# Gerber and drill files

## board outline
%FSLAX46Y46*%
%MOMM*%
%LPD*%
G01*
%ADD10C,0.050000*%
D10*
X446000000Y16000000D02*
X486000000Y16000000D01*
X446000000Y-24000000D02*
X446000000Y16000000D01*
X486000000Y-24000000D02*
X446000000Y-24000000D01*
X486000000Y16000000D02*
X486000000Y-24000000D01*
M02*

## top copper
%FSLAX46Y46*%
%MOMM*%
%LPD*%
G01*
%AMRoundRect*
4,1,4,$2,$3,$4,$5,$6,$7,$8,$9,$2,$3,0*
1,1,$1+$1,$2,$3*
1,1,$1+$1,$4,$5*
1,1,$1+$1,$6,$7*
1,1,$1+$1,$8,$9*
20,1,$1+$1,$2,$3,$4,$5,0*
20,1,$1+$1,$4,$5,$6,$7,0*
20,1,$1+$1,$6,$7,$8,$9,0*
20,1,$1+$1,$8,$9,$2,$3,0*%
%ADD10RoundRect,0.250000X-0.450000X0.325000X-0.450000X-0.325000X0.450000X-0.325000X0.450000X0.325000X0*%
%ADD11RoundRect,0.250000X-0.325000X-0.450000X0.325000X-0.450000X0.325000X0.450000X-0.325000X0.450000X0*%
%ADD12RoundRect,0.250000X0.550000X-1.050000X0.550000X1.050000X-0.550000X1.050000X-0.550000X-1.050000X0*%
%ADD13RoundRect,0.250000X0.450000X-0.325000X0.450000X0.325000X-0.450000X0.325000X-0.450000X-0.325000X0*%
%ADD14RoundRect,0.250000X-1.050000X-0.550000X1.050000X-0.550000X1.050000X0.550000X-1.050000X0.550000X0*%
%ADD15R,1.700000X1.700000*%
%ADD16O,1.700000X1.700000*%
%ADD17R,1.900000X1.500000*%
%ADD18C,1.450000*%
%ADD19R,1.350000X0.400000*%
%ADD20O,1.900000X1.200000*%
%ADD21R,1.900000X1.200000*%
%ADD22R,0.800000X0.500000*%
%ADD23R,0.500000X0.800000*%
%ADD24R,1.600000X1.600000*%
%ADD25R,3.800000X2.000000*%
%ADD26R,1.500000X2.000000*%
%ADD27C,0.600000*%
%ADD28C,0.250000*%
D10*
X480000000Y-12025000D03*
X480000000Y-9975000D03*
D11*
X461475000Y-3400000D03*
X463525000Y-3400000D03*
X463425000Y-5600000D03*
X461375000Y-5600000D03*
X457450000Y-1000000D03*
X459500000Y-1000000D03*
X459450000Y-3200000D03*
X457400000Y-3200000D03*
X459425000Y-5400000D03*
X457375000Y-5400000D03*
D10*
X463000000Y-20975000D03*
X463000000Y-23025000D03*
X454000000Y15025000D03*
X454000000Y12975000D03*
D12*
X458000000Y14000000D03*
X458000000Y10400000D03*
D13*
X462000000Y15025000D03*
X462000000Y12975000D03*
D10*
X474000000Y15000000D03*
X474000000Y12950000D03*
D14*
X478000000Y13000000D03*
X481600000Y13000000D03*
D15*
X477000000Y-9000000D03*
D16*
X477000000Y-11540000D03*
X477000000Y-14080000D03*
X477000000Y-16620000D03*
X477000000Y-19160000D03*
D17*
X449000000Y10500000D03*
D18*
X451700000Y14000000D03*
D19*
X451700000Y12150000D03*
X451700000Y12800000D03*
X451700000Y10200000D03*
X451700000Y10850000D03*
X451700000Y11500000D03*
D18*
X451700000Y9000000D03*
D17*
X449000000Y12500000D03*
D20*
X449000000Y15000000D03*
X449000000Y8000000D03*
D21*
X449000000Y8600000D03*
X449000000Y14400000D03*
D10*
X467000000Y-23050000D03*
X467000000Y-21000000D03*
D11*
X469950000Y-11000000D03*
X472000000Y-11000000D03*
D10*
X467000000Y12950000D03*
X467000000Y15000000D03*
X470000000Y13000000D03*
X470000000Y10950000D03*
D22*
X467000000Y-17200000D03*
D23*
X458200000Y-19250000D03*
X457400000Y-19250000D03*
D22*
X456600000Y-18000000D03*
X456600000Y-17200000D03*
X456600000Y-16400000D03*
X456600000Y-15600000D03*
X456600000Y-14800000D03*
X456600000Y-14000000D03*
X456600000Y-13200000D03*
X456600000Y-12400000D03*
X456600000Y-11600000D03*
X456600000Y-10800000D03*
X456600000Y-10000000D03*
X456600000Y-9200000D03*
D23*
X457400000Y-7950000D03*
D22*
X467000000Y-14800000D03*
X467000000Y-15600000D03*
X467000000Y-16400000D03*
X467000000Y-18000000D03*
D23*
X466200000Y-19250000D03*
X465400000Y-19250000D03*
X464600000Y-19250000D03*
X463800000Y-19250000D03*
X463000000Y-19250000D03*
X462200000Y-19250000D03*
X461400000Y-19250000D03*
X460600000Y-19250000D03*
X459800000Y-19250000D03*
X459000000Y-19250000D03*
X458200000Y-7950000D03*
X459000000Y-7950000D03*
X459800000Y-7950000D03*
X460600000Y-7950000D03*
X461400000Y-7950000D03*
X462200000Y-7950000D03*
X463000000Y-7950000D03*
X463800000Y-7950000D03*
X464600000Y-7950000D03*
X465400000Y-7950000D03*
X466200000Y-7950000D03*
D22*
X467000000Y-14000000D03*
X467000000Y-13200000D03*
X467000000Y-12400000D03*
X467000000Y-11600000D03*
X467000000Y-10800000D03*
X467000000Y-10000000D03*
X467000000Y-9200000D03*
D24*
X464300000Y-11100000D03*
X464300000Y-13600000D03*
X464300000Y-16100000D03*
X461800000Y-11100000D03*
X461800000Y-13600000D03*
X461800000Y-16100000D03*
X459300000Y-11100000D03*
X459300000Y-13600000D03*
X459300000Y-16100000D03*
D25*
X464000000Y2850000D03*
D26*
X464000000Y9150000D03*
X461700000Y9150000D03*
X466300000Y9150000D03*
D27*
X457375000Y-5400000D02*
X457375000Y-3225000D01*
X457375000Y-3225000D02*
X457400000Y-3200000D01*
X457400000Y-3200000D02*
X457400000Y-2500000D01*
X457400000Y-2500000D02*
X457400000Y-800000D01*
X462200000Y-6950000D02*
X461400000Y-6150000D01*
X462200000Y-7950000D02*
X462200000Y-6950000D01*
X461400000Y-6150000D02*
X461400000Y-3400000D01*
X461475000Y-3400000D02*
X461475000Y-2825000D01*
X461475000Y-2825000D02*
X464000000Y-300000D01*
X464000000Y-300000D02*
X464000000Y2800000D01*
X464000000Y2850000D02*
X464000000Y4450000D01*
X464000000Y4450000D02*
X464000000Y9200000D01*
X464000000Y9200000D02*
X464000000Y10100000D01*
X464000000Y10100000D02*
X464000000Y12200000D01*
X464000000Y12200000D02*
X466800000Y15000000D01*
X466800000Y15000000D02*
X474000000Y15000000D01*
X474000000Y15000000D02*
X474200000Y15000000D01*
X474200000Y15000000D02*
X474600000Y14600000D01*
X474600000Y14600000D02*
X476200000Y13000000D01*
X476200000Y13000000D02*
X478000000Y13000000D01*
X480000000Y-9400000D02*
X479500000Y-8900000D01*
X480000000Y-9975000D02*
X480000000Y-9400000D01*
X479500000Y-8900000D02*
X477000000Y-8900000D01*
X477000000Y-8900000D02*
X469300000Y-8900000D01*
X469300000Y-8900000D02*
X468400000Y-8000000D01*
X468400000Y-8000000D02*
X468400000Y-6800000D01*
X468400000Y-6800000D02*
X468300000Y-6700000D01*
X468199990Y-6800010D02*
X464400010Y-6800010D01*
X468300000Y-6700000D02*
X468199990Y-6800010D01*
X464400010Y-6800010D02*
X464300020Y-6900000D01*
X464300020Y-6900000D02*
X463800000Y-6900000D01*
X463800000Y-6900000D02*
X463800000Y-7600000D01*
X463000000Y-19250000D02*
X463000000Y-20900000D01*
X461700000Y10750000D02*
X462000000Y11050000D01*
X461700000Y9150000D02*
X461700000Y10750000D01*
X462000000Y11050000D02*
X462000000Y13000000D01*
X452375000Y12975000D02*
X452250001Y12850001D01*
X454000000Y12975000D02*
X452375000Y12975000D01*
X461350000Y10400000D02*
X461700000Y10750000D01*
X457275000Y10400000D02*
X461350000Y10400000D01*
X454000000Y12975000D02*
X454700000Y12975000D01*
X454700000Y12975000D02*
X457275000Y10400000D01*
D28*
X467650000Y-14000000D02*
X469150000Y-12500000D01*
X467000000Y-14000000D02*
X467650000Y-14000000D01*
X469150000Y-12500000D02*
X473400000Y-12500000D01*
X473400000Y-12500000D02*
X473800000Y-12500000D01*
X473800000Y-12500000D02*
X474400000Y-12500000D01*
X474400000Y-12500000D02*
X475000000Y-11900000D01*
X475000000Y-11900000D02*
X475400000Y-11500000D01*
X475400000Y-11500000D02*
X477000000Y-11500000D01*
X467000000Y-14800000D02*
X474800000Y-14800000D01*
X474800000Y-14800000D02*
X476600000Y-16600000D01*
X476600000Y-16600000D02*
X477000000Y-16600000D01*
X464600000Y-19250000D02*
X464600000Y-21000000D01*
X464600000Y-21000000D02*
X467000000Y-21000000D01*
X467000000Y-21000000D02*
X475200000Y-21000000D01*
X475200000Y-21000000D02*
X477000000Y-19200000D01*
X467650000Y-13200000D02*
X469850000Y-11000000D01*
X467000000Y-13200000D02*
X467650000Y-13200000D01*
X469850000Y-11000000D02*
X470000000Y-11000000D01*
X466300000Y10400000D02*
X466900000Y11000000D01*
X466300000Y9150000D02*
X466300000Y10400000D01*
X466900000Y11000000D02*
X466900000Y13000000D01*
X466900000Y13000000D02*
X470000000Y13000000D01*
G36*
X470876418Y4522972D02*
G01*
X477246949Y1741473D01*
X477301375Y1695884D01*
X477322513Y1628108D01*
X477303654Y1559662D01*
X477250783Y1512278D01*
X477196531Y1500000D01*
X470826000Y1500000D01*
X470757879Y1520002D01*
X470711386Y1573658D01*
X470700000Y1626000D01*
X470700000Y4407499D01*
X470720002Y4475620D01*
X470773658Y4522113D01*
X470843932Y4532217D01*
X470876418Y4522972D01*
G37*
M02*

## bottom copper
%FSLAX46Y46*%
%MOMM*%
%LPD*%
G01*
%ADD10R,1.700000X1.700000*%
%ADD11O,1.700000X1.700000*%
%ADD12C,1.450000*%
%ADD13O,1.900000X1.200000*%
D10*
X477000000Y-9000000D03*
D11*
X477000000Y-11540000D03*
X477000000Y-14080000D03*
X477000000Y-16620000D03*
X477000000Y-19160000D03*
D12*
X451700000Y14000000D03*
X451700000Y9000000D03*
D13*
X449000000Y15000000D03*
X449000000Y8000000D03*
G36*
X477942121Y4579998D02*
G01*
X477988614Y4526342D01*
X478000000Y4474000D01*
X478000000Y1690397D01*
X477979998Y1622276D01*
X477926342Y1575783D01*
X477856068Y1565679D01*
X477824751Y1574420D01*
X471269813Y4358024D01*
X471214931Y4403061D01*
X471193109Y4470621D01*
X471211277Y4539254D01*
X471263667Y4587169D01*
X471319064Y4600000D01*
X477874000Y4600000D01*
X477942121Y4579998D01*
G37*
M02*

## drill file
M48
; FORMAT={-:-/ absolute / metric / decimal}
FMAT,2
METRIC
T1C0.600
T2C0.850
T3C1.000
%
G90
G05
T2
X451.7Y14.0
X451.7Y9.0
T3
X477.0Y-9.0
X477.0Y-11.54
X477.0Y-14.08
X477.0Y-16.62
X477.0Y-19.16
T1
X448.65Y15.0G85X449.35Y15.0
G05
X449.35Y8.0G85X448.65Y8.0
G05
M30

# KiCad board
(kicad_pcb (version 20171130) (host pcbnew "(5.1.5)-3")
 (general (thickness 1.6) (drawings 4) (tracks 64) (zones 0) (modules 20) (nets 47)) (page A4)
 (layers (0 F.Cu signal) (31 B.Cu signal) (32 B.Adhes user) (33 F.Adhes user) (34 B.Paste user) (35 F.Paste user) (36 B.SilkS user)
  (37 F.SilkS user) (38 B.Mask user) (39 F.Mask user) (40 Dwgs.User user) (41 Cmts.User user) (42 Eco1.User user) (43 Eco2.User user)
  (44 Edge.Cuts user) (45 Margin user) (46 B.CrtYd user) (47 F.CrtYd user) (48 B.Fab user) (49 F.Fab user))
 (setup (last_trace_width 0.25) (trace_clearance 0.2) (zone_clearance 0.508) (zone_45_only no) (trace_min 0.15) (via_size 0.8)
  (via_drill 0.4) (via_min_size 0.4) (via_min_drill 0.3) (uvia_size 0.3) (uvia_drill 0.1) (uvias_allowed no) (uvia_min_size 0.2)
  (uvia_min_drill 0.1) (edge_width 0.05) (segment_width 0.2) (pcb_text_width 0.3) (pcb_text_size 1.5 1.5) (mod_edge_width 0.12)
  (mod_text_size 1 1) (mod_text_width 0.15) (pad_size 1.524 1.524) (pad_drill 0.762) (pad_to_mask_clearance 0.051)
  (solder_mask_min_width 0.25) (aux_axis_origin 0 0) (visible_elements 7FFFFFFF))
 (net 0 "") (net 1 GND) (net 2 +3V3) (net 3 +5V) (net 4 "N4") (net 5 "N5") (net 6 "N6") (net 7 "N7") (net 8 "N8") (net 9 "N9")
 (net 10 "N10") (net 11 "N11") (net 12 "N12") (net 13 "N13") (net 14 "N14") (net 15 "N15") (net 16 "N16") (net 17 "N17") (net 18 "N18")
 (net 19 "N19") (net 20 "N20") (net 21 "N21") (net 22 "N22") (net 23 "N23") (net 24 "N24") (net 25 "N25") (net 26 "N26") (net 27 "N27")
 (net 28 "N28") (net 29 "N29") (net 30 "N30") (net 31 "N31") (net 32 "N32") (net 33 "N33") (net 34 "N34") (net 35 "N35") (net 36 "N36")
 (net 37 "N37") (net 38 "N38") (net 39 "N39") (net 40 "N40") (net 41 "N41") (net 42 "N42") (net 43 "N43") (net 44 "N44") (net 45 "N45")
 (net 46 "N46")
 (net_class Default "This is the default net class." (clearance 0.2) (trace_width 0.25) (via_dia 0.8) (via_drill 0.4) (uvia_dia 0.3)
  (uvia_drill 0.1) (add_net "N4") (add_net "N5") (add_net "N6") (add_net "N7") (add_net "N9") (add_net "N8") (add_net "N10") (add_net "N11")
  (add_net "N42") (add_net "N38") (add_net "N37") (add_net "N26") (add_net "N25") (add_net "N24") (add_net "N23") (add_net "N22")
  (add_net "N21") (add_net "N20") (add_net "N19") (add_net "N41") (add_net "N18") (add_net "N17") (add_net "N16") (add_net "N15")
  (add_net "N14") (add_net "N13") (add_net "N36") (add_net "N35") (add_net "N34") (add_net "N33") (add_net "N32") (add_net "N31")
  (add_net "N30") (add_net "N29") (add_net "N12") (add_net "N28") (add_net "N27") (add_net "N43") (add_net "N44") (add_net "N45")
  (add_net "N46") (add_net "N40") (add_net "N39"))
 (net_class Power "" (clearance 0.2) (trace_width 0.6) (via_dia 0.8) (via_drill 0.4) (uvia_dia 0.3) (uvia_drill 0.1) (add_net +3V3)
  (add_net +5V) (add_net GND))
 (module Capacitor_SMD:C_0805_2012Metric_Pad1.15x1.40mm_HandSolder (layer F.Cu) (at 480 11 270)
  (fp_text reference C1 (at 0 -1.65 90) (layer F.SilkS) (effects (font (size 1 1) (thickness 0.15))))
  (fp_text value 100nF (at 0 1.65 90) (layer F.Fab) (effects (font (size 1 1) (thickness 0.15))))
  (pad 2 smd roundrect (at 1.025 0 270) (size 1.15 1.4) (layers F.Cu F.Paste F.Mask) (roundrect_rratio 0.217391) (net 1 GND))
  (pad 1 smd roundrect (at -1.025 0 270) (size 1.15 1.4) (layers F.Cu F.Paste F.Mask) (roundrect_rratio 0.217391) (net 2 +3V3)))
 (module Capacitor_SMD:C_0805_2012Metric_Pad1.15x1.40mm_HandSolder (layer F.Cu) (at 462.5 3.4)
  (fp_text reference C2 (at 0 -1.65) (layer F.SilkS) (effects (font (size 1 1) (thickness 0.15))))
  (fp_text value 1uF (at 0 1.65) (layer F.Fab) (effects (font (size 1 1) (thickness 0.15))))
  (pad 1 smd roundrect (at -1.025 0) (size 1.15 1.4) (layers F.Cu F.Paste F.Mask) (roundrect_rratio 0.217391) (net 2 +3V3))
  (pad 2 smd roundrect (at 1.025 0) (size 1.15 1.4) (layers F.Cu F.Paste F.Mask) (roundrect_rratio 0.217391) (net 1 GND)))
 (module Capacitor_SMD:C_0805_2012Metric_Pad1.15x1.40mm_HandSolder (layer F.Cu) (at 462.4 5.6)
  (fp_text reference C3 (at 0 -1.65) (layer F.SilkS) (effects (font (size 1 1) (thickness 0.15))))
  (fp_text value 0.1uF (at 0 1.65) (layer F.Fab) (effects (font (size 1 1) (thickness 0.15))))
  (pad 2 smd roundrect (at 1.025 0) (size 1.15 1.4) (layers F.Cu F.Paste F.Mask) (roundrect_rratio 0.217391) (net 1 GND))
  (pad 1 smd roundrect (at -1.025 0) (size 1.15 1.4) (layers F.Cu F.Paste F.Mask) (roundrect_rratio 0.217391) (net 2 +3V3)))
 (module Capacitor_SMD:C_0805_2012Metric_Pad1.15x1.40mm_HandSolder (layer F.Cu) (at 458.475 1)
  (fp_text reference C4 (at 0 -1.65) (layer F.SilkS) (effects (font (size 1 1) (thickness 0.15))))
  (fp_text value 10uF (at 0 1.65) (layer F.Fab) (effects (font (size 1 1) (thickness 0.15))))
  (pad 1 smd roundrect (at -1.025 0) (size 1.15 1.4) (layers F.Cu F.Paste F.Mask) (roundrect_rratio 0.217391) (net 2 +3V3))
  (pad 2 smd roundrect (at 1.025 0) (size 1.15 1.4) (layers F.Cu F.Paste F.Mask) (roundrect_rratio 0.217391) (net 1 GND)))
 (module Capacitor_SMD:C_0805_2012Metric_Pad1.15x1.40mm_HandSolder (layer F.Cu) (at 458.425 3.2)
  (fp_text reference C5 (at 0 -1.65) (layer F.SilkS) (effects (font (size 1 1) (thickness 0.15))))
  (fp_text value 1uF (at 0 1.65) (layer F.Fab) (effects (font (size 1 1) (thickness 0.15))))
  (pad 2 smd roundrect (at 1.025 0) (size 1.15 1.4) (layers F.Cu F.Paste F.Mask) (roundrect_rratio 0.217391) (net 1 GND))
  (pad 1 smd roundrect (at -1.025 0) (size 1.15 1.4) (layers F.Cu F.Paste F.Mask) (roundrect_rratio 0.217391) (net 2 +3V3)))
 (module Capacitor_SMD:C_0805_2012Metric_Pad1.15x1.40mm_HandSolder (layer F.Cu) (at 458.4 5.4)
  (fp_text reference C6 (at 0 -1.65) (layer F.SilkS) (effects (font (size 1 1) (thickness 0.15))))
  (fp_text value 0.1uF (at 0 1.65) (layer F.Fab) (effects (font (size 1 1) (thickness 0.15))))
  (pad 2 smd roundrect (at 1.025 0) (size 1.15 1.4) (layers F.Cu F.Paste F.Mask) (roundrect_rratio 0.217391) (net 1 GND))
  (pad 1 smd roundrect (at -1.025 0) (size 1.15 1.4) (layers F.Cu F.Paste F.Mask) (roundrect_rratio 0.217391) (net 2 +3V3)))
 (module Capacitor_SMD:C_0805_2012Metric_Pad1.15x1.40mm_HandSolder (layer F.Cu) (at 463 22 270)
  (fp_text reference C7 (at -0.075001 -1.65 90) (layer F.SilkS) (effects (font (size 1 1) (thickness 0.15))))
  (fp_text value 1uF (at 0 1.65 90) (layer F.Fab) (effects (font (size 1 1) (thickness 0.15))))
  (pad 1 smd roundrect (at -1.025 0 270) (size 1.15 1.4) (layers F.Cu F.Paste F.Mask) (roundrect_rratio 0.217391) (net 2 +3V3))
  (pad 2 smd roundrect (at 1.025 0 270) (size 1.15 1.4) (layers F.Cu F.Paste F.Mask) (roundrect_rratio 0.217391) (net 1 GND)))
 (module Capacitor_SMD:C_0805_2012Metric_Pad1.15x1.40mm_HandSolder (layer F.Cu) (at 454 -14 270)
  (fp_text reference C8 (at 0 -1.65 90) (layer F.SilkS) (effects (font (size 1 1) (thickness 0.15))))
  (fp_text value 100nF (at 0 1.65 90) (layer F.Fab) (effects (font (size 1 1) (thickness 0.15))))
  (pad 1 smd roundrect (at -1.025 0 270) (size 1.15 1.4) (layers F.Cu F.Paste F.Mask) (roundrect_rratio 0.217391) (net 1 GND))
  (pad 2 smd roundrect (at 1.025 0 270) (size 1.15 1.4) (layers F.Cu F.Paste F.Mask) (roundrect_rratio 0.217391) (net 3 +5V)))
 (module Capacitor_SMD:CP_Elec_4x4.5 (layer F.Cu) (at 458 -12.2 90)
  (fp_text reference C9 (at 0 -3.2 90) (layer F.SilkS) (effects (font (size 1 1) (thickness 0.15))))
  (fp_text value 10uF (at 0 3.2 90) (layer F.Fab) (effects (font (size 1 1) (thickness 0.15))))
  (pad 2 smd roundrect (at 1.8 0 90) (size 2.6 1.6) (layers F.Cu F.Paste F.Mask) (roundrect_rratio 0.15625) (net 1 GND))
  (pad 1 smd roundrect (at -1.8 0 90) (size 2.6 1.6) (layers F.Cu F.Paste F.Mask) (roundrect_rratio 0.15625) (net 3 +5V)))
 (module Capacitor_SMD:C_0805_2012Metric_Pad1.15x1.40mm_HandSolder (layer F.Cu) (at 462 -14 90)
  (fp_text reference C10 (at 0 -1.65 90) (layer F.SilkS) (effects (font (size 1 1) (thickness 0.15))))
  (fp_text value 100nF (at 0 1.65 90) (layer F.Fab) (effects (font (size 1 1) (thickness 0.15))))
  (pad 2 smd roundrect (at 1.025 0 90) (size 1.15 1.4) (layers F.Cu F.Paste F.Mask) (roundrect_rratio 0.217391) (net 1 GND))
  (pad 1 smd roundrect (at -1.025 0 90) (size 1.15 1.4) (layers F.Cu F.Paste F.Mask) (roundrect_rratio 0.217391) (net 3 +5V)))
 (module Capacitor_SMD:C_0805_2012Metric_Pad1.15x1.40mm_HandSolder (layer F.Cu) (at 474 -13.975 270)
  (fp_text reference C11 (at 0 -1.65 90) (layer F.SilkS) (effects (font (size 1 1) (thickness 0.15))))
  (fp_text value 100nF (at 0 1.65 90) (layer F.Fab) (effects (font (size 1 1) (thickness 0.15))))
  (pad 1 smd roundrect (at -1.025 0 270) (size 1.15 1.4) (layers F.Cu F.Paste F.Mask) (roundrect_rratio 0.217391) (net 2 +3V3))
  (pad 2 smd roundrect (at 1.025 0 270) (size 1.15 1.4) (layers F.Cu F.Paste F.Mask) (roundrect_rratio 0.217391) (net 1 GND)))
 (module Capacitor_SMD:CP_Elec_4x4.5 (layer F.Cu) (at 479.8 -13)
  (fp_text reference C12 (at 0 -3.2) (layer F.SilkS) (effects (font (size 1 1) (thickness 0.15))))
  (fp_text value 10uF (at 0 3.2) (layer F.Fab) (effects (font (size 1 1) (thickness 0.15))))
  (pad 1 smd roundrect (at -1.8 0) (size 2.6 1.6) (layers F.Cu F.Paste F.Mask) (roundrect_rratio 0.15625) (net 2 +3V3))
  (pad 2 smd roundrect (at 1.8 0) (size 2.6 1.6) (layers F.Cu F.Paste F.Mask) (roundrect_rratio 0.15625) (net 1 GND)))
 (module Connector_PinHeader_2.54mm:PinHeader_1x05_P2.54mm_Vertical (layer F.Cu) (at 477 9)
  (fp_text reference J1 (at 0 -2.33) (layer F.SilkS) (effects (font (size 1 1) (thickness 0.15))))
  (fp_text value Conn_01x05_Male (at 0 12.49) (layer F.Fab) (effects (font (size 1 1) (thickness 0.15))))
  (pad 1 thru_hole rect (at 0 0) (size 1.7 1.7) (drill 1) (layers *.Cu *.Mask) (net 2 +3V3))
  (pad 2 thru_hole oval (at 0 2.54) (size 1.7 1.7) (drill 1) (layers *.Cu *.Mask) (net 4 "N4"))
  (pad 3 thru_hole oval (at 0 5.08) (size 1.7 1.7) (drill 1) (layers *.Cu *.Mask) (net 1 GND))
  (pad 4 thru_hole oval (at 0 7.62) (size 1.7 1.7) (drill 1) (layers *.Cu *.Mask) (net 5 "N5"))
  (pad 5 thru_hole oval (at 0 10.16) (size 1.7 1.7) (drill 1) (layers *.Cu *.Mask) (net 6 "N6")))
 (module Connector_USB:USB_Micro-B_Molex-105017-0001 (layer F.Cu) (at 450.2375 -11.5 270)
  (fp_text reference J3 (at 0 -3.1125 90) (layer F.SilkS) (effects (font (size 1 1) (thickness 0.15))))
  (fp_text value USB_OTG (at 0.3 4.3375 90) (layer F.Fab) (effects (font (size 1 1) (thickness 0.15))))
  (pad 6 smd rect (at 1 1.2375 270) (size 1.5 1.9) (layers F.Cu F.Paste F.Mask) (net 1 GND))
  (pad 6 thru_hole circle (at -2.5 -1.4625 270) (size 1.45 1.45) (drill 0.85) (layers *.Cu *.Mask) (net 1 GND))
  (pad 2 smd rect (at -0.65 -1.4625 270) (size 0.4 1.35) (layers F.Cu F.Paste F.Mask) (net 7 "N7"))
  (pad 1 smd rect (at -1.3 -1.4625 270) (size 0.4 1.35) (layers F.Cu F.Paste F.Mask) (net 3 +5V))
  (pad 5 smd rect (at 1.3 -1.4625 270) (size 0.4 1.35) (layers F.Cu F.Paste F.Mask) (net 1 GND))
  (pad 4 smd rect (at 0.65 -1.4625 270) (size 0.4 1.35) (layers F.Cu F.Paste F.Mask) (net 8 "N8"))
  (pad 3 smd rect (at 0 -1.4625 270) (size 0.4 1.35) (layers F.Cu F.Paste F.Mask) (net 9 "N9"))
  (pad 6 thru_hole circle (at 2.5 -1.4625 270) (size 1.45 1.45) (drill 0.85) (layers *.Cu *.Mask) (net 1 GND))
  (pad 6 smd rect (at -1 1.2375 270) (size 1.5 1.9) (layers F.Cu F.Paste F.Mask) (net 1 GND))
  (pad 6 thru_hole oval (at -3.5 1.2375 90) (size 1.2 1.9) (drill oval 0.6 1.3) (layers *.Cu *.Mask) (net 1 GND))
  (pad 6 thru_hole oval (at 3.5 1.2375 270) (size 1.2 1.9) (drill oval 0.6 1.3) (layers *.Cu *.Mask) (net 1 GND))
  (pad 6 smd rect (at 2.9 1.2375 270) (size 1.2 1.9) (layers F.Cu F.Mask) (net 1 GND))
  (pad 6 smd rect (at -2.9 1.2375 270) (size 1.2 1.9) (layers F.Cu F.Mask) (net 1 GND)))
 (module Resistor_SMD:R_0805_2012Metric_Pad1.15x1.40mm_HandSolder (layer F.Cu) (at 467 22.025 270)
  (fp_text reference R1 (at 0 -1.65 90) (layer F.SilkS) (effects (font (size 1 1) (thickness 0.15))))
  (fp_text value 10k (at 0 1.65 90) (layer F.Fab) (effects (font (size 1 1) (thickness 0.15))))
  (pad 2 smd roundrect (at 1.025 0 270) (size 1.15 1.4) (layers F.Cu F.Paste F.Mask) (roundrect_rratio 0.217391) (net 1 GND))
  (pad 1 smd roundrect (at -1.025 0 270) (size 1.15 1.4) (layers F.Cu F.Paste F.Mask) (roundrect_rratio 0.217391) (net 6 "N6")))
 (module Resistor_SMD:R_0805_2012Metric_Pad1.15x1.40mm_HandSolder (layer F.Cu) (at 470.975 11)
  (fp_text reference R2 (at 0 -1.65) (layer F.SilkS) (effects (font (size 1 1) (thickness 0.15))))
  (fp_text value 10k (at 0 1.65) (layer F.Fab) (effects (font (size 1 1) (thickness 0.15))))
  (pad 1 smd roundrect (at -1.025 0) (size 1.15 1.4) (layers F.Cu F.Paste F.Mask) (roundrect_rratio 0.217391) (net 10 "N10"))
  (pad 2 smd roundrect (at 1.025 0) (size 1.15 1.4) (layers F.Cu F.Paste F.Mask) (roundrect_rratio 0.217391) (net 1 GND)))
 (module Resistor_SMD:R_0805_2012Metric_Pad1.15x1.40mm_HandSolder (layer F.Cu) (at 467 -13.975 270)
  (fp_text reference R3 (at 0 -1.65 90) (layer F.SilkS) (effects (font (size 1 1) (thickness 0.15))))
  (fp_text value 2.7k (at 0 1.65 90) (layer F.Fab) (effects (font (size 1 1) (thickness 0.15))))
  (pad 2 smd roundrect (at 1.025 0 270) (size 1.15 1.4) (layers F.Cu F.Paste F.Mask) (roundrect_rratio 0.217391) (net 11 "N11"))
  (pad 1 smd roundrect (at -1.025 0 270) (size 1.15 1.4) (layers F.Cu F.Paste F.Mask) (roundrect_rratio 0.217391) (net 2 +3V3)))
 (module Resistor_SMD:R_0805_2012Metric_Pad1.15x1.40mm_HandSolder (layer F.Cu) (at 470 -11.975 270)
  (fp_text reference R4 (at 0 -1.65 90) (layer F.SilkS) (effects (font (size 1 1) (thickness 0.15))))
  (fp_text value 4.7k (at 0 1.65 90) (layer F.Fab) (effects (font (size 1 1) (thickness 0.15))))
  (pad 1 smd roundrect (at -1.025 0 270) (size 1.15 1.4) (layers F.Cu F.Paste F.Mask) (roundrect_rratio 0.217391) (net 11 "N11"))
  (pad 2 smd roundrect (at 1.025 0 270) (size 1.15 1.4) (layers F.Cu F.Paste F.Mask) (roundrect_rratio 0.217391) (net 1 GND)))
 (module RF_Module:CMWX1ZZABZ (layer F.Cu) (at 461.8 13.6 270)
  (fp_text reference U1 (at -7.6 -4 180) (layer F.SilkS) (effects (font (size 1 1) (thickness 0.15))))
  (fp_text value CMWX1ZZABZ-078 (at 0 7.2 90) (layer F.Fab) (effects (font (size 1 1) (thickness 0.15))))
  (pad 38 smd rect (at 3.6 -5.2) (size 0.8 0.5) (layers F.Cu F.Paste F.Mask) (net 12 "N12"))
  (pad 26 smd rect (at 5.65 3.6 270) (size 0.8 0.5) (layers F.Cu F.Paste F.Mask) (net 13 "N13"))
  (pad 25 smd rect (at 5.65 4.4 270) (size 0.8 0.5) (layers F.Cu F.Paste F.Mask) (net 1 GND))
  (pad 24 smd rect (at 4.4 5.2 180) (size 0.8 0.5) (layers F.Cu F.Paste F.Mask) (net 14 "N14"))
  (pad 23 smd rect (at 3.6 5.2 180) (size 0.8 0.5) (layers F.Cu F.Paste F.Mask) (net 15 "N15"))
  (pad 22 smd rect (at 2.8 5.2 180) (size 0.8 0.5) (layers F.Cu F.Paste F.Mask) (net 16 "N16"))
  (pad 21 smd rect (at 2 5.2 180) (size 0.8 0.5) (layers F.Cu F.Paste F.Mask) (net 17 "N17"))
  (pad 20 smd rect (at 1.2 5.2 180) (size 0.8 0.5) (layers F.Cu F.Paste F.Mask) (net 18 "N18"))
  (pad 19 smd rect (at 0.4 5.2) (size 0.8 0.5) (layers F.Cu F.Paste F.Mask) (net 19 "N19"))
  (pad 18 smd rect (at -0.4 5.2) (size 0.8 0.5) (layers F.Cu F.Paste F.Mask) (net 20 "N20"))
  (pad 17 smd rect (at -1.2 5.2) (size 0.8 0.5) (layers F.Cu F.Paste F.Mask) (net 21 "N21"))
  (pad 16 smd rect (at -2 5.2) (size 0.8 0.5) (layers F.Cu F.Paste F.Mask) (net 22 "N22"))
  (pad 15 smd rect (at -2.8 5.2) (size 0.8 0.5) (layers F.Cu F.Paste F.Mask) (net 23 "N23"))
  (pad 14 smd rect (at -3.6 5.2) (size 0.8 0.5) (layers F.Cu F.Paste F.Mask) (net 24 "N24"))
  (pad 13 smd rect (at -4.4 5.2) (size 0.8 0.5) (layers F.Cu F.Paste F.Mask) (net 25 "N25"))
  (pad 12 smd rect (at -5.65 4.4 270) (size 0.8 0.5) (layers F.Cu F.Paste F.Mask) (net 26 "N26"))
  (pad 41 smd rect (at 1.2 -5.2) (size 0.8 0.5) (layers F.Cu F.Paste F.Mask) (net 5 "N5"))
  (pad 40 smd rect (at 2 -5.2) (size 0.8 0.5) (layers F.Cu F.Paste F.Mask) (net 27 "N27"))
  (pad 39 smd rect (at 2.8 -5.2) (size 0.8 0.5) (layers F.Cu F.Paste F.Mask) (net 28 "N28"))
  (pad 37 smd rect (at 4.4 -5.2) (size 0.8 0.5) (layers F.Cu F.Paste F.Mask) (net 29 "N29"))
  (pad 36 smd rect (at 5.65 -4.4 270) (size 0.8 0.5) (layers F.Cu F.Paste F.Mask) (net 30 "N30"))
  (pad 35 smd rect (at 5.65 -3.6 270) (size 0.8 0.5) (layers F.Cu F.Paste F.Mask) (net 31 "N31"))
  (pad 34 smd rect (at 5.65 -2.8 270) (size 0.8 0.5) (layers F.Cu F.Paste F.Mask) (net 6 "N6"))
  (pad 33 smd rect (at 5.65 -2 270) (size 0.8 0.5) (layers F.Cu F.Paste F.Mask) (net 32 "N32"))
  (pad 32 smd rect (at 5.65 -1.2 270) (size 0.8 0.5) (layers F.Cu F.Paste F.Mask) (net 2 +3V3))
  (pad 31 smd rect (at 5.65 -0.4 270) (size 0.8 0.5) (layers F.Cu F.Paste F.Mask) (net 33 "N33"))
  (pad 30 smd rect (at 5.65 0.4 270) (size 0.8 0.5) (layers F.Cu F.Paste F.Mask) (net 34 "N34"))
  (pad 29 smd rect (at 5.65 1.2 270) (size 0.8 0.5) (layers F.Cu F.Paste F.Mask) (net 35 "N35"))
  (pad 28 smd rect (at 5.65 2 270) (size 0.8 0.5) (layers F.Cu F.Paste F.Mask) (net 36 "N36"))
  (pad 27 smd rect (at 5.65 2.8 270) (size 0.8 0.5) (layers F.Cu F.Paste F.Mask) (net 1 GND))
  (pad 11 smd rect (at -5.65 3.6 270) (size 0.8 0.5) (layers F.Cu F.Paste F.Mask) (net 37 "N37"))
  (pad 10 smd rect (at -5.65 2.8 270) (size 0.8 0.5) (layers F.Cu F.Paste F.Mask) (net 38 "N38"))
  (pad 9 smd rect (at -5.65 2 270) (size 0.8 0.5) (layers F.Cu F.Paste F.Mask) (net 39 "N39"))
  (pad 8 smd rect (at -5.65 1.2 270) (size 0.8 0.5) (layers F.Cu F.Paste F.Mask) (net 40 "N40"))
  (pad 7 smd rect (at -5.65 0.4 270) (size 0.8 0.5) (layers F.Cu F.Paste F.Mask) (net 1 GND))
  (pad 6 smd rect (at -5.65 -0.4 270) (size 0.8 0.5) (layers F.Cu F.Paste F.Mask) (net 2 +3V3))
  (pad 5 smd rect (at -5.65 -1.2 270) (size 0.8 0.5) (layers F.Cu F.Paste F.Mask) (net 2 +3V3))
  (pad 4 smd rect (at -5.65 -2 270) (size 0.8 0.5) (layers F.Cu F.Paste F.Mask) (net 2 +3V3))
  (pad 3 smd rect (at -5.65 -2.8 270) (size 0.8 0.5) (layers F.Cu F.Paste F.Mask) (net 1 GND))
  (pad 2 smd rect (at -5.65 -3.6 270) (size 0.8 0.5) (layers F.Cu F.Paste F.Mask) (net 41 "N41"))
  (pad 1 smd rect (at -5.65 -4.4 270) (size 0.8 0.5) (layers F.Cu F.Paste F.Mask) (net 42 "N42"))
  (pad 42 smd rect (at 0.4 -5.2) (size 0.8 0.5) (layers F.Cu F.Paste F.Mask) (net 4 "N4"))
  (pad 43 smd rect (at -0.4 -5.2) (size 0.8 0.5) (layers F.Cu F.Paste F.Mask) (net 10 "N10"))
  (pad 44 smd rect (at -1.2 -5.2) (size 0.8 0.5) (layers F.Cu F.Paste F.Mask) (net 1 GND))
  (pad 45 smd rect (at -2 -5.2) (size 0.8 0.5) (layers F.Cu F.Paste F.Mask) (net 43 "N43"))
  (pad 46 smd rect (at -2.8 -5.2) (size 0.8 0.5) (layers F.Cu F.Paste F.Mask) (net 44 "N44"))
  (pad 47 smd rect (at -3.6 -5.2) (size 0.8 0.5) (layers F.Cu F.Paste F.Mask) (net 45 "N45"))
  (pad 48 smd rect (at -4.4 -5.2) (size 0.8 0.5) (layers F.Cu F.Paste F.Mask) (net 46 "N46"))
  (pad 49 smd rect (at -2.5 -2.5) (size 1.6 1.6) (layers F.Cu F.Paste F.Mask) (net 1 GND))
  (pad 50 smd rect (at 0 -2.5) (size 1.6 1.6) (layers F.Cu F.Paste F.Mask) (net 1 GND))
  (pad 51 smd rect (at 2.5 -2.5) (size 1.6 1.6) (layers F.Cu F.Paste F.Mask) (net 1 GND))
  (pad 52 smd rect (at -2.5 0) (size 1.6 1.6) (layers F.Cu F.Paste F.Mask) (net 1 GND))
  (pad 53 smd rect (at 0 0) (size 1.6 1.6) (layers F.Cu F.Paste F.Mask) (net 1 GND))
  (pad 54 smd rect (at 2.5 0) (size 1.6 1.6) (layers F.Cu F.Paste F.Mask) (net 1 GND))
  (pad 55 smd rect (at -2.5 2.5) (size 1.6 1.6) (layers F.Cu F.Paste F.Mask) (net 1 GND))
  (pad 56 smd rect (at 0 2.5) (size 1.6 1.6) (layers F.Cu F.Paste F.Mask) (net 1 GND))
  (pad 57 smd rect (at 2.5 2.5) (size 1.6 1.6) (layers F.Cu F.Paste F.Mask) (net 1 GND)))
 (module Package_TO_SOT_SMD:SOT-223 (layer F.Cu) (at 464 -6 270)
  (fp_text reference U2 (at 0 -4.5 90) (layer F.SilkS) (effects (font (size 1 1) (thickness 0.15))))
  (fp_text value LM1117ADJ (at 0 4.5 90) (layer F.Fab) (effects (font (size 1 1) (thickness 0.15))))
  (pad 4 smd rect (at 3.15 0 270) (size 2 3.8) (layers F.Cu F.Paste F.Mask) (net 2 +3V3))
  (pad 2 smd rect (at -3.15 0 270) (size 2 1.5) (layers F.Cu F.Paste F.Mask) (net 2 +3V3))
  (pad 3 smd rect (at -3.15 2.3 270) (size 2 1.5) (layers F.Cu F.Paste F.Mask) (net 3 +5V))
  (pad 1 smd rect (at -3.15 -2.3 270) (size 2 1.5) (layers F.Cu F.Paste F.Mask) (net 11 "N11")))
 (gr_line (start 446 -16) (end 486 -16) (layer Edge.Cuts) (width 0.05))
 (gr_line (start 446 24) (end 446 -16) (layer Edge.Cuts) (width 0.05))
 (gr_line (start 486 24) (end 446 24) (layer Edge.Cuts) (width 0.05))
 (gr_line (start 486 -16) (end 486 24) (layer Edge.Cuts) (width 0.05))
 (segment (start 457.375 5.4) (end 457.375 3.225) (width 0.6) (layer F.Cu) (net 2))
 (segment (start 457.375 3.225) (end 457.4 3.2) (width 0.6) (layer F.Cu) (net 2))
 (segment (start 457.4 3.2) (end 457.4 2.5) (width 0.6) (layer F.Cu) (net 2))
 (segment (start 457.4 2.5) (end 457.4 0.8) (width 0.6) (layer F.Cu) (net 2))
 (segment (start 462.2 6.95) (end 461.4 6.15) (width 0.6) (layer F.Cu) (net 2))
 (segment (start 462.2 7.95) (end 462.2 6.95) (width 0.6) (layer F.Cu) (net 2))
 (segment (start 461.4 6.15) (end 461.4 3.4) (width 0.6) (layer F.Cu) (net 2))
 (segment (start 461.475 3.4) (end 461.475 2.825) (width 0.6) (layer F.Cu) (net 2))
 (segment (start 461.475 2.825) (end 464 0.3) (width 0.6) (layer F.Cu) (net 2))
 (segment (start 464 0.3) (end 464 -2.8) (width 0.6) (layer F.Cu) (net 2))
 (segment (start 464 -2.85) (end 464 -4.45) (width 0.6) (layer F.Cu) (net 2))
 (segment (start 464 -4.45) (end 464 -9.2) (width 0.6) (layer F.Cu) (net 2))
 (segment (start 464 -9.2) (end 464 -10.1) (width 0.6) (layer F.Cu) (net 2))
 (segment (start 464 -10.1) (end 464 -12.2) (width 0.6) (layer F.Cu) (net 2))
 (segment (start 464 -12.2) (end 466.8 -15) (width 0.6) (layer F.Cu) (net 2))
 (segment (start 466.8 -15) (end 474 -15) (width 0.6) (layer F.Cu) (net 2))
 (segment (start 474 -15) (end 474.2 -15) (width 0.6) (layer F.Cu) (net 2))
 (segment (start 474.2 -15) (end 474.6 -14.6) (width 0.6) (layer F.Cu) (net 2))
 (segment (start 474.6 -14.6) (end 476.2 -13) (width 0.6) (layer F.Cu) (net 2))
 (segment (start 476.2 -13) (end 478 -13) (width 0.6) (layer F.Cu) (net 2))
 (segment (start 480 9.4) (end 479.5 8.9) (width 0.6) (layer F.Cu) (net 2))
 (segment (start 480 9.975) (end 480 9.4) (width 0.6) (layer F.Cu) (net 2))
 (segment (start 479.5 8.9) (end 477 8.9) (width 0.6) (layer F.Cu) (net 2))
 (segment (start 477 8.9) (end 469.3 8.9) (width 0.6) (layer F.Cu) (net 2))
 (segment (start 469.3 8.9) (end 468.4 8) (width 0.6) (layer F.Cu) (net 2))
 (segment (start 468.4 8) (end 468.4 6.8) (width 0.6) (layer F.Cu) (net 2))
 (segment (start 468.4 6.8) (end 468.3 6.7) (width 0.6) (layer F.Cu) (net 2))
 (segment (start 468.19999 6.80001) (end 464.40001 6.80001) (width 0.6) (layer F.Cu) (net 2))
 (segment (start 468.3 6.7) (end 468.19999 6.80001) (width 0.6) (layer F.Cu) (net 2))
 (segment (start 464.40001 6.80001) (end 464.30002 6.9) (width 0.6) (layer F.Cu) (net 2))
 (segment (start 464.30002 6.9) (end 463.8 6.9) (width 0.6) (layer F.Cu) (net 2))
 (segment (start 463.8 6.9) (end 463.8 7.6) (width 0.6) (layer F.Cu) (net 2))
 (segment (start 463 19.25) (end 463 20.9) (width 0.6) (layer F.Cu) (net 2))
 (segment (start 461.7 -10.75) (end 462 -11.05) (width 0.6) (layer F.Cu) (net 3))
 (segment (start 461.7 -9.15) (end 461.7 -10.75) (width 0.6) (layer F.Cu) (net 3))
 (segment (start 462 -11.05) (end 462 -13) (width 0.6) (layer F.Cu) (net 3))
 (segment (start 452.375 -12.975) (end 452.250001 -12.850001) (width 0.6) (layer F.Cu) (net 3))
 (segment (start 454 -12.975) (end 452.375 -12.975) (width 0.6) (layer F.Cu) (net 3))
 (segment (start 461.35 -10.4) (end 461.7 -10.75) (width 0.6) (layer F.Cu) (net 3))
 (segment (start 457.275 -10.4) (end 461.35 -10.4) (width 0.6) (layer F.Cu) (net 3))
 (segment (start 454 -12.975) (end 454.7 -12.975) (width 0.6) (layer F.Cu) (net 3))
 (segment (start 454.7 -12.975) (end 457.275 -10.4) (width 0.6) (layer F.Cu) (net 3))
 (segment (start 467.65 14) (end 469.15 12.5) (width 0.25) (layer F.Cu) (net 4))
 (segment (start 467 14) (end 467.65 14) (width 0.25) (layer F.Cu) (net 4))
 (segment (start 469.15 12.5) (end 473.4 12.5) (width 0.25) (layer F.Cu) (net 4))
 (segment (start 473.4 12.5) (end 473.8 12.5) (width 0.25) (layer F.Cu) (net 4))
 (segment (start 473.8 12.5) (end 474.4 12.5) (width 0.25) (layer F.Cu) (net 4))
 (segment (start 474.4 12.5) (end 475 11.9) (width 0.25) (layer F.Cu) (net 4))
 (segment (start 475 11.9) (end 475.4 11.5) (width 0.25) (layer F.Cu) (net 4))
 (segment (start 475.4 11.5) (end 477 11.5) (width 0.25) (layer F.Cu) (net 4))
 (segment (start 467 14.8) (end 474.8 14.8) (width 0.25) (layer F.Cu) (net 5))
 (segment (start 474.8 14.8) (end 476.6 16.6) (width 0.25) (layer F.Cu) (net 5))
 (segment (start 476.6 16.6) (end 477 16.6) (width 0.25) (layer F.Cu) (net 5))
 (segment (start 464.6 19.25) (end 464.6 21) (width 0.25) (layer F.Cu) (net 6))
 (segment (start 464.6 21) (end 467 21) (width 0.25) (layer F.Cu) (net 6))
 (segment (start 467 21) (end 475.2 21) (width 0.25) (layer F.Cu) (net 6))
 (segment (start 475.2 21) (end 477 19.2) (width 0.25) (layer F.Cu) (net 6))
 (segment (start 467.65 13.2) (end 469.85 11) (width 0.25) (layer F.Cu) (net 10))
 (segment (start 467 13.2) (end 467.65 13.2) (width 0.25) (layer F.Cu) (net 10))
 (segment (start 469.85 11) (end 470 11) (width 0.25) (layer F.Cu) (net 10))
 (segment (start 466.3 -10.4) (end 466.9 -11) (width 0.25) (layer F.Cu) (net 11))
 (segment (start 466.3 -9.15) (end 466.3 -10.4) (width 0.25) (layer F.Cu) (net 11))
 (segment (start 466.9 -11) (end 466.9 -13) (width 0.25) (layer F.Cu) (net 11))
 (segment (start 466.9 -13) (end 470 -13) (width 0.25) (layer F.Cu) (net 11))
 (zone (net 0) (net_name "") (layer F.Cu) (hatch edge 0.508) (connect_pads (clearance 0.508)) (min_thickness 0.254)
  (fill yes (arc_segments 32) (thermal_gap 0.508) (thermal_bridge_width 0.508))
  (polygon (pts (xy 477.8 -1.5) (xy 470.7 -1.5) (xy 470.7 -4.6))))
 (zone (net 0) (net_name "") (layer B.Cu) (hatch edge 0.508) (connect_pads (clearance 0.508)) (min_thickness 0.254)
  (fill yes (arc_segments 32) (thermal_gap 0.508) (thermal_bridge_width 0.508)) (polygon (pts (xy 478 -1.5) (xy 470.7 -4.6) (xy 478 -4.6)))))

